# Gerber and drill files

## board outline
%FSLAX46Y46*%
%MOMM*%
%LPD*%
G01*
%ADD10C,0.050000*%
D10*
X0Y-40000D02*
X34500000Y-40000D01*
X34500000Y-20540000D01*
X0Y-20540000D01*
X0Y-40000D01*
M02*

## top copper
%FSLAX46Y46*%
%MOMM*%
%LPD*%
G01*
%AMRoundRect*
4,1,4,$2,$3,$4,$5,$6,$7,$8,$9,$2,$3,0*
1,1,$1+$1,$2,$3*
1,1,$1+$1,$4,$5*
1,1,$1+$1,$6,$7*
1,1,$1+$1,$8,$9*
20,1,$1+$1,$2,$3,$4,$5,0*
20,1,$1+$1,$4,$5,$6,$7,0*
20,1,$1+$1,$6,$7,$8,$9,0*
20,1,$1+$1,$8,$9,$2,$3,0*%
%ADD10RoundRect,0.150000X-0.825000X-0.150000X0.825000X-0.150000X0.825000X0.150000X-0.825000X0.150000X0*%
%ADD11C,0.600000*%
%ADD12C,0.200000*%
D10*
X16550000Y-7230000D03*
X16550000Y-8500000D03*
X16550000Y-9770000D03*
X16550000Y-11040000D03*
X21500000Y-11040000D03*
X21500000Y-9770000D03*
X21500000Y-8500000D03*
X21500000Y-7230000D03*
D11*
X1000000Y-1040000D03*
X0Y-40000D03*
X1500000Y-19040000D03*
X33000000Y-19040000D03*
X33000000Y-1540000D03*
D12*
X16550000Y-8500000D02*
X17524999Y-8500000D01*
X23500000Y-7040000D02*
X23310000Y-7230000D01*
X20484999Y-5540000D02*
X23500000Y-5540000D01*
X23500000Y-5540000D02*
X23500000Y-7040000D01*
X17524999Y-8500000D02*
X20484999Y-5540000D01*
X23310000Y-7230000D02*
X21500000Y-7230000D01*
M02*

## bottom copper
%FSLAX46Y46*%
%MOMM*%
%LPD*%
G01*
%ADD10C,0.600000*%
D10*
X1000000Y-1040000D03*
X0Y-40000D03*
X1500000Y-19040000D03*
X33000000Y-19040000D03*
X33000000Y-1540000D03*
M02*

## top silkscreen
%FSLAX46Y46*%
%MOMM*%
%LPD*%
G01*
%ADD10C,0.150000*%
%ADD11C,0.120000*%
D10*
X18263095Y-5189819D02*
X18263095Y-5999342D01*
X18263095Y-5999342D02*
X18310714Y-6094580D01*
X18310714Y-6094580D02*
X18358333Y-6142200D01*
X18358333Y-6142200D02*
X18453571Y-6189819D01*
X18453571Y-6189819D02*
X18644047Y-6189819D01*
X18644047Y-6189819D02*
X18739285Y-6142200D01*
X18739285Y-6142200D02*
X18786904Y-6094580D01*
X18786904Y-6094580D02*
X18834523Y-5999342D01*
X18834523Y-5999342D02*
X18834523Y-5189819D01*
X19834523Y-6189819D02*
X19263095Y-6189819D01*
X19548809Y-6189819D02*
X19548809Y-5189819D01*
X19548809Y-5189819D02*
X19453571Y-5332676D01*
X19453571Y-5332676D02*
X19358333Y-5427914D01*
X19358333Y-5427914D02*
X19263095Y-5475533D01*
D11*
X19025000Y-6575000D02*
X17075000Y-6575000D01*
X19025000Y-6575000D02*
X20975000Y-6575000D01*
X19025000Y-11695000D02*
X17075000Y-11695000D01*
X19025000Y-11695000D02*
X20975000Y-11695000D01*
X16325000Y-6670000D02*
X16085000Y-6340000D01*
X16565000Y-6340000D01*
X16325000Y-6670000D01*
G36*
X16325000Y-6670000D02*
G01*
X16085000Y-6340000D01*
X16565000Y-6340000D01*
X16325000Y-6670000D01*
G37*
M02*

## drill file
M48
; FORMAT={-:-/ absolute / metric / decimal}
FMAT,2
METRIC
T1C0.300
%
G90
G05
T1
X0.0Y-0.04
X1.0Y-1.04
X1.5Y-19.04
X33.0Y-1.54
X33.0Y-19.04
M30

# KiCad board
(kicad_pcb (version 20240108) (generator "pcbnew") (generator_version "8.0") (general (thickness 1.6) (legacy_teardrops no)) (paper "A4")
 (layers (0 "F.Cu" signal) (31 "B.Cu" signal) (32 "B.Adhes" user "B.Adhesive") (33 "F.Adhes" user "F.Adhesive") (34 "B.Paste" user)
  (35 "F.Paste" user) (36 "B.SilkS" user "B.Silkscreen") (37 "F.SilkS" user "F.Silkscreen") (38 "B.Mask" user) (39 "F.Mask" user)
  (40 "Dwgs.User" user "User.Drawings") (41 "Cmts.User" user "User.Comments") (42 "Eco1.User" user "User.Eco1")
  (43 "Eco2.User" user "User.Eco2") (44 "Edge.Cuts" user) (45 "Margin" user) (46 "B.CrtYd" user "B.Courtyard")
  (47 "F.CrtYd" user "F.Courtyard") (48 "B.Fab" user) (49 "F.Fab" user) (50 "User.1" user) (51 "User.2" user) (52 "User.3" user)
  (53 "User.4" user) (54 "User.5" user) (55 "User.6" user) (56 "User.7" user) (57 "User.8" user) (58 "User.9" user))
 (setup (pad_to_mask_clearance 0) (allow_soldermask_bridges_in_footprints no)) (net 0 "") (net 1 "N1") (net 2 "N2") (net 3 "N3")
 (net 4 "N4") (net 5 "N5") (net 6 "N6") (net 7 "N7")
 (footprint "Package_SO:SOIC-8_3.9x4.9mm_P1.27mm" (layer "F.Cu") (at 19.025 9.135)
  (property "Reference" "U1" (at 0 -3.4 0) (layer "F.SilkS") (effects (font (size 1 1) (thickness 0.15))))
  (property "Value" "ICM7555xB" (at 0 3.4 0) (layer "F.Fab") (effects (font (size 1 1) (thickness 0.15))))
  (fp_line (start 0 -2.56) (end -1.95 -2.56) (stroke (width 0.12) (type solid)) (layer "F.SilkS"))
  (fp_line (start 0 -2.56) (end 1.95 -2.56) (stroke (width 0.12) (type solid)) (layer "F.SilkS"))
  (fp_line (start 0 2.56) (end -1.95 2.56) (stroke (width 0.12) (type solid)) (layer "F.SilkS"))
  (fp_line (start 0 2.56) (end 1.95 2.56) (stroke (width 0.12) (type solid)) (layer "F.SilkS"))
  (fp_poly
   (pts (xy -2.7 -2.465) (xy -2.94 -2.795) (xy -2.46 -2.795) (xy -2.7 -2.465)) (stroke (width 0.12) (type solid)) (fill solid)
   (layer "F.SilkS"))
  (pad "1" smd roundrect (at -2.475 -1.905) (size 1.95 0.6) (layers "F.Cu" "F.Paste" "F.Mask") (roundrect_rratio 0.25) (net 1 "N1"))
  (pad "2" smd roundrect (at -2.475 -0.635) (size 1.95 0.6) (layers "F.Cu" "F.Paste" "F.Mask") (roundrect_rratio 0.25) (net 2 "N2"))
  (pad "3" smd roundrect (at -2.475 0.635) (size 1.95 0.6) (layers "F.Cu" "F.Paste" "F.Mask") (roundrect_rratio 0.25) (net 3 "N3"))
  (pad "4" smd roundrect (at -2.475 1.905) (size 1.95 0.6) (layers "F.Cu" "F.Paste" "F.Mask") (roundrect_rratio 0.25) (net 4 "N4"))
  (pad "5" smd roundrect (at 2.475 1.905) (size 1.95 0.6) (layers "F.Cu" "F.Paste" "F.Mask") (roundrect_rratio 0.25) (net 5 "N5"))
  (pad "6" smd roundrect (at 2.475 0.635) (size 1.95 0.6) (layers "F.Cu" "F.Paste" "F.Mask") (roundrect_rratio 0.25) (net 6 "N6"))
  (pad "7" smd roundrect (at 2.475 -0.635) (size 1.95 0.6) (layers "F.Cu" "F.Paste" "F.Mask") (roundrect_rratio 0.25) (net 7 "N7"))
  (pad "8" smd roundrect (at 2.475 -1.905) (size 1.95 0.6) (layers "F.Cu" "F.Paste" "F.Mask") (roundrect_rratio 0.25) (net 2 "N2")))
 (gr_rect (start 0 0.04) (end 34.5 20.54) (stroke (width 0.05) (type default)) (fill none) (layer "Edge.Cuts"))
 (via (at 1 1.04) (size 0.6) (drill 0.3) (layers "F.Cu" "B.Cu") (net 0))
 (via (at 0 0.04) (size 0.6) (drill 0.3) (layers "F.Cu" "B.Cu") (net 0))
 (via (at 1.5 19.04) (size 0.6) (drill 0.3) (layers "F.Cu" "B.Cu") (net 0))
 (via (at 33 19.04) (size 0.6) (drill 0.3) (layers "F.Cu" "B.Cu") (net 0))
 (via (at 33 1.54) (size 0.6) (drill 0.3) (layers "F.Cu" "B.Cu") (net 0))
 (segment (start 16.55 8.5) (end 17.524999 8.5) (width 0.2) (layer "F.Cu") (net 2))
 (segment (start 23.5 7.04) (end 23.31 7.23) (width 0.2) (layer "F.Cu") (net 2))
 (segment (start 20.484999 5.54) (end 23.5 5.54) (width 0.2) (layer "F.Cu") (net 2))
 (segment (start 23.5 5.54) (end 23.5 7.04) (width 0.2) (layer "F.Cu") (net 2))
 (segment (start 17.524999 8.5) (end 20.484999 5.54) (width 0.2) (layer "F.Cu") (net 2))
 (segment (start 23.31 7.23) (end 21.5 7.23) (width 0.2) (layer "F.Cu") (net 2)))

